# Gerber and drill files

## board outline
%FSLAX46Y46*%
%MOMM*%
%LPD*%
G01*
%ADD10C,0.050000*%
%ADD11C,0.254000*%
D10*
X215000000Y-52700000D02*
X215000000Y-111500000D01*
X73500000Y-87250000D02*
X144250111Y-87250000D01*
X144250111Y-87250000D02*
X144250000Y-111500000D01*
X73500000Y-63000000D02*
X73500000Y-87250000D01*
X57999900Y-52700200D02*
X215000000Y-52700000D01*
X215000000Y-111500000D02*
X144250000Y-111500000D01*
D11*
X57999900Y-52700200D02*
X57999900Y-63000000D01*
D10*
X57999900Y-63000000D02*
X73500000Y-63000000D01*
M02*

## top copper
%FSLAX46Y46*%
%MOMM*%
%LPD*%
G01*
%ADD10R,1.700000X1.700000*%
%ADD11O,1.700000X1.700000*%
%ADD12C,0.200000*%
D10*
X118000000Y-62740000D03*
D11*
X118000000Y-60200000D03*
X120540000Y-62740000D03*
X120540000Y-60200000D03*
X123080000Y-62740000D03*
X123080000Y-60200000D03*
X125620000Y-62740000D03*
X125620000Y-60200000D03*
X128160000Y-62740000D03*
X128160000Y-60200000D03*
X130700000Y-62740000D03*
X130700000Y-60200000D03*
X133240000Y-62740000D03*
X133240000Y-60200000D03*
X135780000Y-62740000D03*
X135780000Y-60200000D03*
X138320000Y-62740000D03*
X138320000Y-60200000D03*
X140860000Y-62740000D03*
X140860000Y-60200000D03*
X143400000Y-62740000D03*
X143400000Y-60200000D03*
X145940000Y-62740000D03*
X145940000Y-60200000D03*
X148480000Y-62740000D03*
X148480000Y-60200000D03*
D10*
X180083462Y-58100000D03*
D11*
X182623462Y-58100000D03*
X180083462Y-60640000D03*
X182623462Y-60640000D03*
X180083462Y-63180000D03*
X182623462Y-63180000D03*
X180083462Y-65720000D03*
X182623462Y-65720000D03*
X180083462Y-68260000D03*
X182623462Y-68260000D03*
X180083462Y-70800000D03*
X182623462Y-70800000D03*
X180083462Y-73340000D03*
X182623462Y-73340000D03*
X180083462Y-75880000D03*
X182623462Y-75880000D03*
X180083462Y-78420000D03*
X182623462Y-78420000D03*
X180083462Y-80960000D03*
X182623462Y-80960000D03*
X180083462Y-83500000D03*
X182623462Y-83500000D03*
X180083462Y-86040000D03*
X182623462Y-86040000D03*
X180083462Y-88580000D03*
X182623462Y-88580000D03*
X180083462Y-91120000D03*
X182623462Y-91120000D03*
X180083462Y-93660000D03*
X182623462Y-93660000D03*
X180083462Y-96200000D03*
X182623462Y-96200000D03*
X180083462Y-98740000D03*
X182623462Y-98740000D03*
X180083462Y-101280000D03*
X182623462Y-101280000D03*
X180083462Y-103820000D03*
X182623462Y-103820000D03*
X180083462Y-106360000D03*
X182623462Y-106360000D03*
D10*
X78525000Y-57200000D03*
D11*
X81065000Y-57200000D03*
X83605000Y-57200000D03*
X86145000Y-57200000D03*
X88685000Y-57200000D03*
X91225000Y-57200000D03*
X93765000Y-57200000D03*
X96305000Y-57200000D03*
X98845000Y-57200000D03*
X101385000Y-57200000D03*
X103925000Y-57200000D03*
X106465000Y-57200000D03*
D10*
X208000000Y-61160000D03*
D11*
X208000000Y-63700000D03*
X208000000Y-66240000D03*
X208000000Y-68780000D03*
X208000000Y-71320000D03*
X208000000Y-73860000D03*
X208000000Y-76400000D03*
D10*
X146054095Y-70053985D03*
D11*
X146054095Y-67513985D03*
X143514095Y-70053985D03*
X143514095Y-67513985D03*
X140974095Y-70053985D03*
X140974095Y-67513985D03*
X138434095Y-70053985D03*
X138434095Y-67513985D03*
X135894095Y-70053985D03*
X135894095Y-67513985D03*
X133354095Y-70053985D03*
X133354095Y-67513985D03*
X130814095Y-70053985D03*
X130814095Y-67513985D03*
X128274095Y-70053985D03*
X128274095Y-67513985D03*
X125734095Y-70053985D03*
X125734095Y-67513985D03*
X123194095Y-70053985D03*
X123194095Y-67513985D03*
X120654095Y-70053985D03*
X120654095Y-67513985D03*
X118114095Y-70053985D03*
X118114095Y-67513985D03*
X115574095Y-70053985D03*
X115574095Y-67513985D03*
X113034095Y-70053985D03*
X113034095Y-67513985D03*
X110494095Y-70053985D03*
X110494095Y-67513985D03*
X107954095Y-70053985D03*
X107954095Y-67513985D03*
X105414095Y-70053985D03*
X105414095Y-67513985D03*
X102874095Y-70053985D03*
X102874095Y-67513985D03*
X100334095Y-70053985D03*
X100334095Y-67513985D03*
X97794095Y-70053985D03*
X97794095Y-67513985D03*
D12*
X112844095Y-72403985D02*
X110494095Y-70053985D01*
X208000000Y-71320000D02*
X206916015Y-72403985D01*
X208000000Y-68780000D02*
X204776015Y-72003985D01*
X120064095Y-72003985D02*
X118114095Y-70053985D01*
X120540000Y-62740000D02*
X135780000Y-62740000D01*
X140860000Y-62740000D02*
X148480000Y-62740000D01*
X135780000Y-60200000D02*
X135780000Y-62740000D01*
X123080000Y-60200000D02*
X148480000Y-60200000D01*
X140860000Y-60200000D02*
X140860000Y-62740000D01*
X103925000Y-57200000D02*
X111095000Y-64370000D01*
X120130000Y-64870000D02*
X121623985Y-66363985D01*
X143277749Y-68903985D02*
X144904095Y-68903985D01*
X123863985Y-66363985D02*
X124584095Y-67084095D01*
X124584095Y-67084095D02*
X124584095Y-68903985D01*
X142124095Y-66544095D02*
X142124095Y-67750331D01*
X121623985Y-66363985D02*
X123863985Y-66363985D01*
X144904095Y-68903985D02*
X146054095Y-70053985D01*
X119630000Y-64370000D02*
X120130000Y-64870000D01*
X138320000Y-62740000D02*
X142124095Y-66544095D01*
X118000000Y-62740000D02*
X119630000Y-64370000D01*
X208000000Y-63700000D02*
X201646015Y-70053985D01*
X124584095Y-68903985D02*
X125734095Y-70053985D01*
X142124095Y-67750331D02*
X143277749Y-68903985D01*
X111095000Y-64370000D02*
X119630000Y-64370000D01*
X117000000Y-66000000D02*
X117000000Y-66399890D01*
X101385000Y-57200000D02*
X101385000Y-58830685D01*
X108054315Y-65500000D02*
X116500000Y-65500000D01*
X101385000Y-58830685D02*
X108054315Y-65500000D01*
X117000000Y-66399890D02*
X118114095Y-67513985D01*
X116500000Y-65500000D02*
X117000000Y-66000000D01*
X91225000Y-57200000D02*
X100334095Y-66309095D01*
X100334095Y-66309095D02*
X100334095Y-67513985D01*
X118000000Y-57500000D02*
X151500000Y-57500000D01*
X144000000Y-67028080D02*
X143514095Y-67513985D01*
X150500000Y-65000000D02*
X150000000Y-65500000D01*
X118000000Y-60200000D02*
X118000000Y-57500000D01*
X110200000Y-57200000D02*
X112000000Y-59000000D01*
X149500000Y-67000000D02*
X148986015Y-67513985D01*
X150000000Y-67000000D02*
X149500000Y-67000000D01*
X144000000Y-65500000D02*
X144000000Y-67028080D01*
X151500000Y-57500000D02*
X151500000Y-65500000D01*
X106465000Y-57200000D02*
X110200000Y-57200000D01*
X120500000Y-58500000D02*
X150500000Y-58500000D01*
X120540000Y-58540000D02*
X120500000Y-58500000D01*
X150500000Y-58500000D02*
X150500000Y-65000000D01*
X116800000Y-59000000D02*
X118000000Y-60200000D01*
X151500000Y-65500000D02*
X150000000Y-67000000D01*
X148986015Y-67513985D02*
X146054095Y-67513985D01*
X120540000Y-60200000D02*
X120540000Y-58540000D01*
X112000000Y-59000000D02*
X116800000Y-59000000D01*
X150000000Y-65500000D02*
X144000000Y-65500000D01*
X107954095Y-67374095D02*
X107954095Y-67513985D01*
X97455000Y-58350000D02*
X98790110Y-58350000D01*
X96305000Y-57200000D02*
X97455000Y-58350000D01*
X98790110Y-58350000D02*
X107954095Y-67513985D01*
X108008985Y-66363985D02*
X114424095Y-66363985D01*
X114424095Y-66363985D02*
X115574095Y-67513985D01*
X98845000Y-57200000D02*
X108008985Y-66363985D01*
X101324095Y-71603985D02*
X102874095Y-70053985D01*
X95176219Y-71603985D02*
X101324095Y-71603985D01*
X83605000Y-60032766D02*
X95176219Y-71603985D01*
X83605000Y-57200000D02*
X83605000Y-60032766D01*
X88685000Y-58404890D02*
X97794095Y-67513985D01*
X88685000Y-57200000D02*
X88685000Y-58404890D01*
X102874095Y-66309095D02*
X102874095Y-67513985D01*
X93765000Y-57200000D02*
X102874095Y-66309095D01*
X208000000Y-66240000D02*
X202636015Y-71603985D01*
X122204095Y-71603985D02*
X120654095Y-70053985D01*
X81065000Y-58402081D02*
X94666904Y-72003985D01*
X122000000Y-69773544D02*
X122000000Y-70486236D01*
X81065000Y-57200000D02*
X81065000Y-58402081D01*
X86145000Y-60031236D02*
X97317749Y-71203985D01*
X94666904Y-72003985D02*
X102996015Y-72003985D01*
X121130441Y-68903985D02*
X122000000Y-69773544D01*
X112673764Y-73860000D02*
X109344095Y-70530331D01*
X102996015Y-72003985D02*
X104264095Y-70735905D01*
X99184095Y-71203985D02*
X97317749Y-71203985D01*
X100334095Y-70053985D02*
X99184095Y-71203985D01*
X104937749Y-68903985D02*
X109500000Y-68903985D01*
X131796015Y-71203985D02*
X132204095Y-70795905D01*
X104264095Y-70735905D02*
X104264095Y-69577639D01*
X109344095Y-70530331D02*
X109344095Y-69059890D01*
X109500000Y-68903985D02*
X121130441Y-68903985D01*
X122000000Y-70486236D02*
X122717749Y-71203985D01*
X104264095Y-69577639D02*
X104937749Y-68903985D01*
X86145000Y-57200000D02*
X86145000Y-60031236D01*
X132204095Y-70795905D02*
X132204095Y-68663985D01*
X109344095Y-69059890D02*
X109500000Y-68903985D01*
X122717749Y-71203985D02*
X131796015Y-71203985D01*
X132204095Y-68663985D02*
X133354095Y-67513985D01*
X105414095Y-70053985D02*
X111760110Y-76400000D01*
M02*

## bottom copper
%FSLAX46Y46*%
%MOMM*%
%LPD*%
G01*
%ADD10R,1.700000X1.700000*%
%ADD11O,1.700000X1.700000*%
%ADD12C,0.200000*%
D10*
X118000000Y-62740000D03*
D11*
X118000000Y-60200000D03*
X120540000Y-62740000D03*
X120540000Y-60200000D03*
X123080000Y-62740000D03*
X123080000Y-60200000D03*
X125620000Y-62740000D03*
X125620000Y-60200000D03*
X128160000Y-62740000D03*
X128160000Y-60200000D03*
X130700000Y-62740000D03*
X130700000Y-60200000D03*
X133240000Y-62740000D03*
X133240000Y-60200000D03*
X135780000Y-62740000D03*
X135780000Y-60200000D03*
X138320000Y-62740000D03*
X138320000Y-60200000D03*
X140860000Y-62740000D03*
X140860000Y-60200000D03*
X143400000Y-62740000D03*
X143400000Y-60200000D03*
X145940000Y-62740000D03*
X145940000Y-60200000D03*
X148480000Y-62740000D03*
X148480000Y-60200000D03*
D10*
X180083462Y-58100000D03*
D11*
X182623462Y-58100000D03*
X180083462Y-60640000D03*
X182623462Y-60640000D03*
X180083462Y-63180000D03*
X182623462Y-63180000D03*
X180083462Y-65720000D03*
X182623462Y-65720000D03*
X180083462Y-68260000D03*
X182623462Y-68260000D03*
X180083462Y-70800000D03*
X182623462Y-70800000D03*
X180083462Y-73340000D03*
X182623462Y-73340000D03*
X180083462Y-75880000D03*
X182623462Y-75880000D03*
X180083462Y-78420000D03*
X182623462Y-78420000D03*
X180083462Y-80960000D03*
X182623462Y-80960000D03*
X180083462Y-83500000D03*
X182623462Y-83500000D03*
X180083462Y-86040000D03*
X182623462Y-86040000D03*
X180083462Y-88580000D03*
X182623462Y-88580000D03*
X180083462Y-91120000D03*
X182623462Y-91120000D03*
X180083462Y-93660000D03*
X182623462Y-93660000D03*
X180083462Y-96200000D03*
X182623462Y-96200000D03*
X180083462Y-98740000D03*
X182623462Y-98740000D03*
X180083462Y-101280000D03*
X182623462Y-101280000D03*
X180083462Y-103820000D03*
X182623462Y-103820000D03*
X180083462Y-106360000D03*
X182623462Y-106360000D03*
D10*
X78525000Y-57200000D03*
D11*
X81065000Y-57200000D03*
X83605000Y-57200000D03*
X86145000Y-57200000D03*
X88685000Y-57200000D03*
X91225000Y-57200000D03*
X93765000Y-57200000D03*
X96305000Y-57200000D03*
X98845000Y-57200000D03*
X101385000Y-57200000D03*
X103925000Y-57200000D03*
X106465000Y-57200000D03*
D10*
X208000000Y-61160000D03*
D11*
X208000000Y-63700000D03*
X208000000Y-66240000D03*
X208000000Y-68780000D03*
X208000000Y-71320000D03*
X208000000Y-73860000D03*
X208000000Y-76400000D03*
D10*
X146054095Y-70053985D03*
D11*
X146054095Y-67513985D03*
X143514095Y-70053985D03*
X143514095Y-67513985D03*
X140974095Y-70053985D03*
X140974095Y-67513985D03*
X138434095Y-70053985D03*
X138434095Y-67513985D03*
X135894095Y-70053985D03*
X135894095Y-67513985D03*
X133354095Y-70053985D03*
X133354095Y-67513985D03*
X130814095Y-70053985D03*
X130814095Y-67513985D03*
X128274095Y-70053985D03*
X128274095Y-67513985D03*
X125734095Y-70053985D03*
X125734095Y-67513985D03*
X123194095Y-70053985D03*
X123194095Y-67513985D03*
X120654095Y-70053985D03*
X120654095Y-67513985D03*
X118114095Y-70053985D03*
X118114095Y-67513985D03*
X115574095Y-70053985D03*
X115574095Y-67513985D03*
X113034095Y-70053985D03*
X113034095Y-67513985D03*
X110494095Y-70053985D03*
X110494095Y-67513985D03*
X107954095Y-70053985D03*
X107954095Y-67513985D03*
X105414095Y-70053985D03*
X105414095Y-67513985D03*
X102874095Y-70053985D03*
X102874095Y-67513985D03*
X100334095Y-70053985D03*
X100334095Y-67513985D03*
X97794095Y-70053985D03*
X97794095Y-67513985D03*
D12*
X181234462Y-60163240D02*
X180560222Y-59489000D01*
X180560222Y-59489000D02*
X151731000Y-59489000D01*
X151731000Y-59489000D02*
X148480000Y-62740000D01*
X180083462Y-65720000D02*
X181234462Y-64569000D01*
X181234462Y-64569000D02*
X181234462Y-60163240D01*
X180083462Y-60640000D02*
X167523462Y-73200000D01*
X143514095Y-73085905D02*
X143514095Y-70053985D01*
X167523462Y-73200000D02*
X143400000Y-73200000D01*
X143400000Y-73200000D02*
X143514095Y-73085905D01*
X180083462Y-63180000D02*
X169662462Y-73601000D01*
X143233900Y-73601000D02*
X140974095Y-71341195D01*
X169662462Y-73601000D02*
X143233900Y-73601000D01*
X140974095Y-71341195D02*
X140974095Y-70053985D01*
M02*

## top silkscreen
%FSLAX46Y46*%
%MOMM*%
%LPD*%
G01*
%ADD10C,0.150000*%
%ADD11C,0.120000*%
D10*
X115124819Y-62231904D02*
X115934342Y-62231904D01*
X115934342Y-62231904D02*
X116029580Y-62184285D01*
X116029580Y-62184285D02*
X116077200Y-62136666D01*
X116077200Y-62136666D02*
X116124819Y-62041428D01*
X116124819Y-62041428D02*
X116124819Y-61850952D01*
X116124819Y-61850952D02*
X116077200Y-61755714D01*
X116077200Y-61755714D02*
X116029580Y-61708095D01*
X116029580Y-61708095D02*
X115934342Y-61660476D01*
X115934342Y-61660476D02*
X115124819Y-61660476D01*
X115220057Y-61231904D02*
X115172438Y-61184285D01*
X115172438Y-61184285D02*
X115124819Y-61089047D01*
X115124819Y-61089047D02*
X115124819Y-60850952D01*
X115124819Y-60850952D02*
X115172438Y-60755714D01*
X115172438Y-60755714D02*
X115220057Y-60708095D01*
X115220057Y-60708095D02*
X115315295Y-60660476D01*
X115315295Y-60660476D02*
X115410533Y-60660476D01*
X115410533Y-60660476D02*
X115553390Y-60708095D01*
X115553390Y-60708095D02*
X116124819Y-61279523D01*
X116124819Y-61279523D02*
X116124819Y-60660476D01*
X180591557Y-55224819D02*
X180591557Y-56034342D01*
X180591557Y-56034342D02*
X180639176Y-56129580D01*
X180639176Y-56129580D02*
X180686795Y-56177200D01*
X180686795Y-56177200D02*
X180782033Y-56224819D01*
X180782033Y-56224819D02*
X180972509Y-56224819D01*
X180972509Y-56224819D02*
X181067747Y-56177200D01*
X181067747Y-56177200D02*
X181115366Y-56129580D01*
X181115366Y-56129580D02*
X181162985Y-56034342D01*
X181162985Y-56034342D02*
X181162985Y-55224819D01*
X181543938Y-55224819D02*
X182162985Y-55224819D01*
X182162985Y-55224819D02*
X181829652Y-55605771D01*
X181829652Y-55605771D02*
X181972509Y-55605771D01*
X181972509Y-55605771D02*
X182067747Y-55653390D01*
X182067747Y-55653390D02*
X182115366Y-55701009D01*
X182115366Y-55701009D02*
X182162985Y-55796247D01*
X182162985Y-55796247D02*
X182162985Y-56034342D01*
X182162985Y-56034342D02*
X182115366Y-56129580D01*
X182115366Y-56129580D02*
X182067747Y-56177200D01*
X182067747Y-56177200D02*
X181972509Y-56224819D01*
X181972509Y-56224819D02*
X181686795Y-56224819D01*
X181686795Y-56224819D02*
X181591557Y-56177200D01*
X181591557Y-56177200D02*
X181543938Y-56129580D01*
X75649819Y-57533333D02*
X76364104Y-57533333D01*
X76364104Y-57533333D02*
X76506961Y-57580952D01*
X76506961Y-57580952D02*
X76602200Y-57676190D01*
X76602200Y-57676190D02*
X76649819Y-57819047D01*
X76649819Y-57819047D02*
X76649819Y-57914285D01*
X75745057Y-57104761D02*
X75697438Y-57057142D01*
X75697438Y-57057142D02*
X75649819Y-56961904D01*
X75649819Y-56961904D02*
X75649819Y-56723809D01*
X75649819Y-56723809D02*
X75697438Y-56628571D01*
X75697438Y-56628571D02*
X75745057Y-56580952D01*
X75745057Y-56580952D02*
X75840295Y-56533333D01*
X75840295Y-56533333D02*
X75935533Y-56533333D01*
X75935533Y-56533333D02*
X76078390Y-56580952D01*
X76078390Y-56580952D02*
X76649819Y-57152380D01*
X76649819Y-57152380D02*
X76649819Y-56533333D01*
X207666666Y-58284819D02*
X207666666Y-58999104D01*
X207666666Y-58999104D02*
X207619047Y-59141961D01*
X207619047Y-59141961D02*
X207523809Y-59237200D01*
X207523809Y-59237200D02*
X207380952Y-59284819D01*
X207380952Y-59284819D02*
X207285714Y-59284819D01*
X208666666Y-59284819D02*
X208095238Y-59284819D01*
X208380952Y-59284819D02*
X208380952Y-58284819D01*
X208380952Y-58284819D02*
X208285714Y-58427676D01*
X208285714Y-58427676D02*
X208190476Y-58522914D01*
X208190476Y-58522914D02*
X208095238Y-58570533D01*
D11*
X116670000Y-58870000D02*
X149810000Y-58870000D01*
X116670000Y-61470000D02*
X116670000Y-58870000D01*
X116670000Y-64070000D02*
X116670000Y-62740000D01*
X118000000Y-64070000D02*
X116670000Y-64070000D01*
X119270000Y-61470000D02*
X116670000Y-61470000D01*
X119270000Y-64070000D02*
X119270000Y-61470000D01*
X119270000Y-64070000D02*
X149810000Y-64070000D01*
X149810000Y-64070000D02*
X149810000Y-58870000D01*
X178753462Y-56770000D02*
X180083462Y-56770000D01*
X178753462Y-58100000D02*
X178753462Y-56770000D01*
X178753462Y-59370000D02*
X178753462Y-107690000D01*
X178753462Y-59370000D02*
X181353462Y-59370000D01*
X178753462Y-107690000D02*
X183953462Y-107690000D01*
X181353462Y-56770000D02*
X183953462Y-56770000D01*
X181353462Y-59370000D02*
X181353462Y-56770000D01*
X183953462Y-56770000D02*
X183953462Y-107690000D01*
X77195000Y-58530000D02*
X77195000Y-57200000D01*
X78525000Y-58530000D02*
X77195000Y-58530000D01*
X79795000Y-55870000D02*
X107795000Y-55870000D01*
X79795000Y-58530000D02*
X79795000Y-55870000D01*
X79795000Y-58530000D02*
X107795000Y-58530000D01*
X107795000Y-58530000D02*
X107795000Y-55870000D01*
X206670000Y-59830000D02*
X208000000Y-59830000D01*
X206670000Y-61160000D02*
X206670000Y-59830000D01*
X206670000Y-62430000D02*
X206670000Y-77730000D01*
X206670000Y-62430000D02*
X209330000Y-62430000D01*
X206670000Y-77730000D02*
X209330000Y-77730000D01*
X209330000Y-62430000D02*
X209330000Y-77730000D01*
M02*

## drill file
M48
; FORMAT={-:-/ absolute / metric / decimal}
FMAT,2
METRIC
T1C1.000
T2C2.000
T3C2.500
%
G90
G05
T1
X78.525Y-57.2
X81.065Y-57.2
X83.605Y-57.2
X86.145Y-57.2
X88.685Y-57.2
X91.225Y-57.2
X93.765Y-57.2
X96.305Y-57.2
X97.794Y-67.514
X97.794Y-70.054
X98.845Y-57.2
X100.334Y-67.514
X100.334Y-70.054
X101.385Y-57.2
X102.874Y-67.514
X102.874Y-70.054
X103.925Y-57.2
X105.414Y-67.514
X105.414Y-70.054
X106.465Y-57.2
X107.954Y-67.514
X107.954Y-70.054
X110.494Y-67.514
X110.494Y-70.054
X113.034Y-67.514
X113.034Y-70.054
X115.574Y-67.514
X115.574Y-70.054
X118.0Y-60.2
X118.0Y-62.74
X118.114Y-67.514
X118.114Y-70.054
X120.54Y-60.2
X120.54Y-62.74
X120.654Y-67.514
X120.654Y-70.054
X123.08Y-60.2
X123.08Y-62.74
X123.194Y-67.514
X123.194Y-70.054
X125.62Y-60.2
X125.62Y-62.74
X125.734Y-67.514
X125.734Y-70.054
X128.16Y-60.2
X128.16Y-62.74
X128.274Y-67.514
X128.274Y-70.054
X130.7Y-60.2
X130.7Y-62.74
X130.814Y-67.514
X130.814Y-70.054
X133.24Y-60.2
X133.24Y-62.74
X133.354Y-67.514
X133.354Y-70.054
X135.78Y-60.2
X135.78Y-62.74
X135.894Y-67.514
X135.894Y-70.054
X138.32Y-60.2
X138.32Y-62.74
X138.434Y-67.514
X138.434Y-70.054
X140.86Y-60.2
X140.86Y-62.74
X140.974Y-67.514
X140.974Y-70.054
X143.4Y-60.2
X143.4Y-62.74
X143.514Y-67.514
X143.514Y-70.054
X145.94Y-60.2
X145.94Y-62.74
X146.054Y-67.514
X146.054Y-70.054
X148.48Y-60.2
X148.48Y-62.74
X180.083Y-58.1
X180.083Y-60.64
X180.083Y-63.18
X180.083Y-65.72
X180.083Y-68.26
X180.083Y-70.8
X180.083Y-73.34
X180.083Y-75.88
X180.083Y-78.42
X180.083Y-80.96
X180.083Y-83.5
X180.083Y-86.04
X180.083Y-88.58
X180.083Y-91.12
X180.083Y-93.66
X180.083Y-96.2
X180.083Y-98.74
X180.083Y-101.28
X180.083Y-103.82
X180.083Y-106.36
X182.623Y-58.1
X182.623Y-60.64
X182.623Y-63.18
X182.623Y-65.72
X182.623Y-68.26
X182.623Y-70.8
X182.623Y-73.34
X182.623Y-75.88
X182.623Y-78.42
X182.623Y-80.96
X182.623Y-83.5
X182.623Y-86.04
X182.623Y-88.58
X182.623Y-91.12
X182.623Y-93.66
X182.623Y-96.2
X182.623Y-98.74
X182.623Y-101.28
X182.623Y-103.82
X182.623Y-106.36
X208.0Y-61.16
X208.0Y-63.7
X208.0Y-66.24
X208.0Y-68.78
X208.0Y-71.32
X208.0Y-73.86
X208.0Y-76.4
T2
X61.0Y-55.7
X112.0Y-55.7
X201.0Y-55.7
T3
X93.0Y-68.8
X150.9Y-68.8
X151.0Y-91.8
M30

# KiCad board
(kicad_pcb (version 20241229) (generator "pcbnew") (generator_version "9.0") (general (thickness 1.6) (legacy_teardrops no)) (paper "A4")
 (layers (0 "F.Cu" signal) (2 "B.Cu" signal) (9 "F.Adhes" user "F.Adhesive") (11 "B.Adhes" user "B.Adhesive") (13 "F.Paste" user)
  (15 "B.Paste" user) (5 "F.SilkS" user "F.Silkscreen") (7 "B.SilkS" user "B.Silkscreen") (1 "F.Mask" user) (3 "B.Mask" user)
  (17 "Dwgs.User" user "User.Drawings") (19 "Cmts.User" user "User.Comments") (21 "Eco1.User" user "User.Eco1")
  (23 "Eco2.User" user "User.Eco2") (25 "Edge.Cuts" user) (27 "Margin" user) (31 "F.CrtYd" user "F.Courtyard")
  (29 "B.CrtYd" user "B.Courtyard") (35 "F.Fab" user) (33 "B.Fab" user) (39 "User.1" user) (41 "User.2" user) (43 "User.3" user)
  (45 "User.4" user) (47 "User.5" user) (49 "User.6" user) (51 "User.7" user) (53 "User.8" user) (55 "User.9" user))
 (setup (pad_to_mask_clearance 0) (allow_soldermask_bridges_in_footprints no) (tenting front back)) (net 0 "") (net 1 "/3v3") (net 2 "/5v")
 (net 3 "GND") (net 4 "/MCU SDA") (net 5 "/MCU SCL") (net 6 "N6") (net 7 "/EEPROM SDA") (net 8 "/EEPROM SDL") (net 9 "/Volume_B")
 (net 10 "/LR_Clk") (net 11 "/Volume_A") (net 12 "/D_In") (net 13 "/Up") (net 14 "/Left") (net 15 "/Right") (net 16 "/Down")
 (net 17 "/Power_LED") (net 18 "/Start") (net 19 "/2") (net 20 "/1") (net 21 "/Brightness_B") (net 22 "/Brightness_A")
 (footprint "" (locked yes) (layer "F.Cu") (at 151 91.8)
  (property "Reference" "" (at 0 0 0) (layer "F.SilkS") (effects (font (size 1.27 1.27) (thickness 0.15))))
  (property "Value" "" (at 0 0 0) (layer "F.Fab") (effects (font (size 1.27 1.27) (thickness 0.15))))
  (pad "" np_thru_hole circle (at 0 0 180) (size 2.5 2.5) (drill 2.5) (layers "*.Cu" "*.Mask")))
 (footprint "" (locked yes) (layer "F.Cu") (at 112 55.7)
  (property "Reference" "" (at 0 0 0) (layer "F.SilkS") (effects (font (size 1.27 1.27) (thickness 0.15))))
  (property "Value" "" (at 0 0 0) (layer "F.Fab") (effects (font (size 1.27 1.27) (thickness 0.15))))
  (pad "" np_thru_hole circle (at 0 0 180) (size 2 2) (drill 2) (layers "*.Cu" "*.Mask")))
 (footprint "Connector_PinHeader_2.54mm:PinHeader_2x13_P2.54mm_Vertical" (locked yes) (layer "F.Cu") (at 118 62.74 90)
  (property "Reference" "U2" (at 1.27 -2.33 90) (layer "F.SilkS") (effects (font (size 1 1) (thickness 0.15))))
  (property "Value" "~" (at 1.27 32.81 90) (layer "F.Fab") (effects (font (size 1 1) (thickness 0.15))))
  (fp_line (start 3.87 -1.33) (end 3.87 31.81) (stroke (width 0.12) (type solid)) (layer "F.SilkS"))
  (fp_line (start 1.27 -1.33) (end 3.87 -1.33) (stroke (width 0.12) (type solid)) (layer "F.SilkS"))
  (fp_line (start -1.33 -1.33) (end 0 -1.33) (stroke (width 0.12) (type solid)) (layer "F.SilkS"))
  (fp_line (start -1.33 0) (end -1.33 -1.33) (stroke (width 0.12) (type solid)) (layer "F.SilkS"))
  (fp_line (start 1.27 1.27) (end 1.27 -1.33) (stroke (width 0.12) (type solid)) (layer "F.SilkS"))
  (fp_line (start -1.33 1.27) (end 1.27 1.27) (stroke (width 0.12) (type solid)) (layer "F.SilkS"))
  (fp_line (start -1.33 1.27) (end -1.33 31.81) (stroke (width 0.12) (type solid)) (layer "F.SilkS"))
  (fp_line (start -1.33 31.81) (end 3.87 31.81) (stroke (width 0.12) (type solid)) (layer "F.SilkS"))
  (pad "1" thru_hole rect (at 0 0 90) (size 1.7 1.7) (drill 1) (layers "*.Cu" "*.Mask") (remove_unused_layers no) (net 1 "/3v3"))
  (pad "2" thru_hole oval (at 2.54 0 90) (size 1.7 1.7) (drill 1) (layers "*.Cu" "*.Mask") (remove_unused_layers no) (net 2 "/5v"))
  (pad "3" thru_hole oval (at 0 2.54 90) (size 1.7 1.7) (drill 1) (layers "*.Cu" "*.Mask") (remove_unused_layers no) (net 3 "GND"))
  (pad "4" thru_hole oval (at 2.54 2.54 90) (size 1.7 1.7) (drill 1) (layers "*.Cu" "*.Mask") (remove_unused_layers no) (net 2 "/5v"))
  (pad "5" thru_hole oval (at 0 5.08 90) (size 1.7 1.7) (drill 1) (layers "*.Cu" "*.Mask") (remove_unused_layers no) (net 3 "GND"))
  (pad "6" thru_hole oval (at 2.54 5.08 90) (size 1.7 1.7) (drill 1) (layers "*.Cu" "*.Mask") (remove_unused_layers no) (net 3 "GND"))
  (pad "7" thru_hole oval (at 0 7.62 90) (size 1.7 1.7) (drill 1) (layers "*.Cu" "*.Mask") (remove_unused_layers no) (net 3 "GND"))
  (pad "8" thru_hole oval (at 2.54 7.62 90) (size 1.7 1.7) (drill 1) (layers "*.Cu" "*.Mask") (remove_unused_layers no) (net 3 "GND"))
  (pad "9" thru_hole oval (at 0 10.16 90) (size 1.7 1.7) (drill 1) (layers "*.Cu" "*.Mask") (remove_unused_layers no) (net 3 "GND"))
  (pad "10" thru_hole oval (at 2.54 10.16 90) (size 1.7 1.7) (drill 1) (layers "*.Cu" "*.Mask") (remove_unused_layers no) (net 3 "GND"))
  (pad "11" thru_hole oval (at 0 12.7 90) (size 1.7 1.7) (drill 1) (layers "*.Cu" "*.Mask") (remove_unused_layers no) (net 3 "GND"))
  (pad "12" thru_hole oval (at 2.54 12.7 90) (size 1.7 1.7) (drill 1) (layers "*.Cu" "*.Mask") (remove_unused_layers no) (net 3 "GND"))
  (pad "13" thru_hole oval (at 0 15.24 90) (size 1.7 1.7) (drill 1) (layers "*.Cu" "*.Mask") (remove_unused_layers no) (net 3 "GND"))
  (pad "14" thru_hole oval (at 2.54 15.24 90) (size 1.7 1.7) (drill 1) (layers "*.Cu" "*.Mask") (remove_unused_layers no) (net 3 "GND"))
  (pad "15" thru_hole oval (at 0 17.78 90) (size 1.7 1.7) (drill 1) (layers "*.Cu" "*.Mask") (remove_unused_layers no) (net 3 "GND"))
  (pad "16" thru_hole oval (at 2.54 17.78 90) (size 1.7 1.7) (drill 1) (layers "*.Cu" "*.Mask") (remove_unused_layers no) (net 3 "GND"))
  (pad "17" thru_hole oval (at 0 20.32 90) (size 1.7 1.7) (drill 1) (layers "*.Cu" "*.Mask") (remove_unused_layers no) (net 1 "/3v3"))
  (pad "18" thru_hole oval (at 2.54 20.32 90) (size 1.7 1.7) (drill 1) (layers "*.Cu" "*.Mask") (remove_unused_layers no) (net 3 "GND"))
  (pad "19" thru_hole oval (at 0 22.86 90) (size 1.7 1.7) (drill 1) (layers "*.Cu" "*.Mask") (remove_unused_layers no) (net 3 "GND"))
  (pad "20" thru_hole oval (at 2.54 22.86 90) (size 1.7 1.7) (drill 1) (layers "*.Cu" "*.Mask") (remove_unused_layers no) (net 3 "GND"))
  (pad "21" thru_hole oval (at 0 25.4 90) (size 1.7 1.7) (drill 1) (layers "*.Cu" "*.Mask") (remove_unused_layers no) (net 3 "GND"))
  (pad "22" thru_hole oval (at 2.54 25.4 90) (size 1.7 1.7) (drill 1) (layers "*.Cu" "*.Mask") (remove_unused_layers no) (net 3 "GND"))
  (pad "23" thru_hole oval (at 0 27.94 90) (size 1.7 1.7) (drill 1) (layers "*.Cu" "*.Mask") (remove_unused_layers no) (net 3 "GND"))
  (pad "24" thru_hole oval (at 2.54 27.94 90) (size 1.7 1.7) (drill 1) (layers "*.Cu" "*.Mask") (remove_unused_layers no) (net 3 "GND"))
  (pad "25" thru_hole oval (at 0 30.48 90) (size 1.7 1.7) (drill 1) (layers "*.Cu" "*.Mask") (remove_unused_layers no) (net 3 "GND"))
  (pad "26" thru_hole oval (at 2.54 30.48 90) (size 1.7 1.7) (drill 1) (layers "*.Cu" "*.Mask") (remove_unused_layers no) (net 3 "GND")))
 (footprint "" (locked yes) (layer "F.Cu") (at 93 68.8)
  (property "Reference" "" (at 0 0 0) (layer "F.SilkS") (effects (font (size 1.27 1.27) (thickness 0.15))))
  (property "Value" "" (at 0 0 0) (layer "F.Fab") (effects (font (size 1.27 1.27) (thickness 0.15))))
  (pad "" np_thru_hole circle (at 0 0 180) (size 2.5 2.5) (drill 2.5) (layers "*.Cu" "*.Mask")))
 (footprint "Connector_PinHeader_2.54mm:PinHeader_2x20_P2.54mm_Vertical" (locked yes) (layer "F.Cu") (at 180.083462 58.1)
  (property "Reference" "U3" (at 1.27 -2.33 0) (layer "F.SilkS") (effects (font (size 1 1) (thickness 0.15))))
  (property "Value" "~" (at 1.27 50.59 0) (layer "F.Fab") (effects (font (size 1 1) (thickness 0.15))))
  (fp_line (start -1.33 -1.33) (end 0 -1.33) (stroke (width 0.12) (type solid)) (layer "F.SilkS"))
  (fp_line (start -1.33 0) (end -1.33 -1.33) (stroke (width 0.12) (type solid)) (layer "F.SilkS"))
  (fp_line (start -1.33 1.27) (end -1.33 49.59) (stroke (width 0.12) (type solid)) (layer "F.SilkS"))
  (fp_line (start -1.33 1.27) (end 1.27 1.27) (stroke (width 0.12) (type solid)) (layer "F.SilkS"))
  (fp_line (start -1.33 49.59) (end 3.87 49.59) (stroke (width 0.12) (type solid)) (layer "F.SilkS"))
  (fp_line (start 1.27 -1.33) (end 3.87 -1.33) (stroke (width 0.12) (type solid)) (layer "F.SilkS"))
  (fp_line (start 1.27 1.27) (end 1.27 -1.33) (stroke (width 0.12) (type solid)) (layer "F.SilkS"))
  (fp_line (start 3.87 -1.33) (end 3.87 49.59) (stroke (width 0.12) (type solid)) (layer "F.SilkS"))
  (pad "1" thru_hole rect (at 0 0) (size 1.7 1.7) (drill 1) (layers "*.Cu" "*.Mask") (remove_unused_layers no) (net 1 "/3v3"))
  (pad "2" thru_hole oval (at 2.54 0) (size 1.7 1.7) (drill 1) (layers "*.Cu" "*.Mask") (remove_unused_layers no) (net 2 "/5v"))
  (pad "3" thru_hole oval (at 0 2.54) (size 1.7 1.7) (drill 1) (layers "*.Cu" "*.Mask") (remove_unused_layers no) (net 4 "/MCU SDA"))
  (pad "4" thru_hole oval (at 2.54 2.54) (size 1.7 1.7) (drill 1) (layers "*.Cu" "*.Mask") (remove_unused_layers no) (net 2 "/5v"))
  (pad "5" thru_hole oval (at 0 5.08) (size 1.7 1.7) (drill 1) (layers "*.Cu" "*.Mask") (remove_unused_layers no) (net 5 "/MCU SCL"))
  (pad "6" thru_hole oval (at 2.54 5.08) (size 1.7 1.7) (drill 1) (layers "*.Cu" "*.Mask") (remove_unused_layers no) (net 3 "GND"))
  (pad "7" thru_hole oval (at 0 7.62) (size 1.7 1.7) (drill 1) (layers "*.Cu" "*.Mask") (remove_unused_layers no) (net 3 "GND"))
  (pad "8" thru_hole oval (at 2.54 7.62) (size 1.7 1.7) (drill 1) (layers "*.Cu" "*.Mask") (remove_unused_layers no) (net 3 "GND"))
  (pad "9" thru_hole oval (at 0 10.16) (size 1.7 1.7) (drill 1) (layers "*.Cu" "*.Mask") (remove_unused_layers no) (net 3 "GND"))
  (pad "10" thru_hole oval (at 2.54 10.16) (size 1.7 1.7) (drill 1) (layers "*.Cu" "*.Mask") (remove_unused_layers no) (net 3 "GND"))
  (pad "11" thru_hole oval (at 0 12.7) (size 1.7 1.7) (drill 1) (layers "*.Cu" "*.Mask") (remove_unused_layers no) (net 3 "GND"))
  (pad "12" thru_hole oval (at 2.54 12.7) (size 1.7 1.7) (drill 1) (layers "*.Cu" "*.Mask") (remove_unused_layers no) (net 3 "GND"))
  (pad "13" thru_hole oval (at 0 15.24) (size 1.7 1.7) (drill 1) (layers "*.Cu" "*.Mask") (remove_unused_layers no) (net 3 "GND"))
  (pad "14" thru_hole oval (at 2.54 15.24) (size 1.7 1.7) (drill 1) (layers "*.Cu" "*.Mask") (remove_unused_layers no) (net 3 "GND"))
  (pad "15" thru_hole oval (at 0 17.78) (size 1.7 1.7) (drill 1) (layers "*.Cu" "*.Mask") (remove_unused_layers no) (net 3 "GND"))
  (pad "16" thru_hole oval (at 2.54 17.78) (size 1.7 1.7) (drill 1) (layers "*.Cu" "*.Mask") (remove_unused_layers no) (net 3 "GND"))
  (pad "17" thru_hole oval (at 0 20.32) (size 1.7 1.7) (drill 1) (layers "*.Cu" "*.Mask") (remove_unused_layers no) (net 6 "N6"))
  (pad "18" thru_hole oval (at 2.54 20.32) (size 1.7 1.7) (drill 1) (layers "*.Cu" "*.Mask") (remove_unused_layers no) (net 3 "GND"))
  (pad "19" thru_hole oval (at 0 22.86) (size 1.7 1.7) (drill 1) (layers "*.Cu" "*.Mask") (remove_unused_layers no) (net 3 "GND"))
  (pad "20" thru_hole oval (at 2.54 22.86) (size 1.7 1.7) (drill 1) (layers "*.Cu" "*.Mask") (remove_unused_layers no) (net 3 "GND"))
  (pad "21" thru_hole oval (at 0 25.4) (size 1.7 1.7) (drill 1) (layers "*.Cu" "*.Mask") (remove_unused_layers no) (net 3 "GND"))
  (pad "22" thru_hole oval (at 2.54 25.4) (size 1.7 1.7) (drill 1) (layers "*.Cu" "*.Mask") (remove_unused_layers no) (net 3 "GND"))
  (pad "23" thru_hole oval (at 0 27.94) (size 1.7 1.7) (drill 1) (layers "*.Cu" "*.Mask") (remove_unused_layers no) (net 3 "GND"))
  (pad "24" thru_hole oval (at 2.54 27.94) (size 1.7 1.7) (drill 1) (layers "*.Cu" "*.Mask") (remove_unused_layers no) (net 3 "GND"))
  (pad "25" thru_hole oval (at 0 30.48) (size 1.7 1.7) (drill 1) (layers "*.Cu" "*.Mask") (remove_unused_layers no) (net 3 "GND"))
  (pad "26" thru_hole oval (at 2.54 30.48) (size 1.7 1.7) (drill 1) (layers "*.Cu" "*.Mask") (remove_unused_layers no) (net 3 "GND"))
  (pad "27" thru_hole oval (at 0 33.02) (size 1.7 1.7) (drill 1) (layers "*.Cu" "*.Mask") (remove_unused_layers no) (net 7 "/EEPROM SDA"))
  (pad "28" thru_hole oval (at 2.54 33.02) (size 1.7 1.7) (drill 1) (layers "*.Cu" "*.Mask") (remove_unused_layers no) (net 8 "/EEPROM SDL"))
  (pad "29" thru_hole oval (at 0 35.56) (size 1.7 1.7) (drill 1) (layers "*.Cu" "*.Mask") (remove_unused_layers no) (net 3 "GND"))
  (pad "30" thru_hole oval (at 2.54 35.56) (size 1.7 1.7) (drill 1) (layers "*.Cu" "*.Mask") (remove_unused_layers no) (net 3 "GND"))
  (pad "31" thru_hole oval (at 0 38.1) (size 1.7 1.7) (drill 1) (layers "*.Cu" "*.Mask") (remove_unused_layers no) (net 3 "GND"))
  (pad "32" thru_hole oval (at 2.54 38.1) (size 1.7 1.7) (drill 1) (layers "*.Cu" "*.Mask") (remove_unused_layers no) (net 3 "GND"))
  (pad "33" thru_hole oval (at 0 40.64) (size 1.7 1.7) (drill 1) (layers "*.Cu" "*.Mask") (remove_unused_layers no) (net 3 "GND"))
  (pad "34" thru_hole oval (at 2.54 40.64) (size 1.7 1.7) (drill 1) (layers "*.Cu" "*.Mask") (remove_unused_layers no) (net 3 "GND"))
  (pad "35" thru_hole oval (at 0 43.18) (size 1.7 1.7) (drill 1) (layers "*.Cu" "*.Mask") (remove_unused_layers no) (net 3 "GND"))
  (pad "36" thru_hole oval (at 2.54 43.18) (size 1.7 1.7) (drill 1) (layers "*.Cu" "*.Mask") (remove_unused_layers no) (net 3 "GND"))
  (pad "37" thru_hole oval (at 0 45.72) (size 1.7 1.7) (drill 1) (layers "*.Cu" "*.Mask") (remove_unused_layers no) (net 3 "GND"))
  (pad "38" thru_hole oval (at 2.54 45.72) (size 1.7 1.7) (drill 1) (layers "*.Cu" "*.Mask") (remove_unused_layers no) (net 3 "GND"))
  (pad "39" thru_hole oval (at 0 48.26) (size 1.7 1.7) (drill 1) (layers "*.Cu" "*.Mask") (remove_unused_layers no) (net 3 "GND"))
  (pad "40" thru_hole oval (at 2.54 48.26) (size 1.7 1.7) (drill 1) (layers "*.Cu" "*.Mask") (remove_unused_layers no) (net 3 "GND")))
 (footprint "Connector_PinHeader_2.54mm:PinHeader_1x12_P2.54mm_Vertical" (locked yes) (layer "F.Cu") (at 78.525 57.2 90)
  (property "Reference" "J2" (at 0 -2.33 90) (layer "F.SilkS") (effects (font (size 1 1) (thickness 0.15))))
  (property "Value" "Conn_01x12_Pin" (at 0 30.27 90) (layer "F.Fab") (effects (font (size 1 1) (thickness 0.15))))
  (fp_line (start -1.33 -1.33) (end 0 -1.33) (stroke (width 0.12) (type solid)) (layer "F.SilkS"))
  (fp_line (start -1.33 0) (end -1.33 -1.33) (stroke (width 0.12) (type solid)) (layer "F.SilkS"))
  (fp_line (start 1.33 1.27) (end 1.33 29.27) (stroke (width 0.12) (type solid)) (layer "F.SilkS"))
  (fp_line (start -1.33 1.27) (end 1.33 1.27) (stroke (width 0.12) (type solid)) (layer "F.SilkS"))
  (fp_line (start -1.33 1.27) (end -1.33 29.27) (stroke (width 0.12) (type solid)) (layer "F.SilkS"))
  (fp_line (start -1.33 29.27) (end 1.33 29.27) (stroke (width 0.12) (type solid)) (layer "F.SilkS"))
  (pad "1" thru_hole rect (at 0 0 90) (size 1.7 1.7) (drill 1) (layers "*.Cu" "*.Mask") (remove_unused_layers no) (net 3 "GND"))
  (pad "2" thru_hole oval (at 0 2.54 90) (size 1.7 1.7) (drill 1) (layers "*.Cu" "*.Mask") (remove_unused_layers no) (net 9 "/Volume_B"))
  (pad "3" thru_hole oval (at 0 5.08 90) (size 1.7 1.7) (drill 1) (layers "*.Cu" "*.Mask") (remove_unused_layers no) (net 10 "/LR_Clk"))
  (pad "4" thru_hole oval (at 0 7.62 90) (size 1.7 1.7) (drill 1) (layers "*.Cu" "*.Mask") (remove_unused_layers no) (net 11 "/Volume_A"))
  (pad "5" thru_hole oval (at 0 10.16 90) (size 1.7 1.7) (drill 1) (layers "*.Cu" "*.Mask") (remove_unused_layers no) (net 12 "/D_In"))
  (pad "6" thru_hole oval (at 0 12.7 90) (size 1.7 1.7) (drill 1) (layers "*.Cu" "*.Mask") (remove_unused_layers no) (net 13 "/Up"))
  (pad "7" thru_hole oval (at 0 15.24 90) (size 1.7 1.7) (drill 1) (layers "*.Cu" "*.Mask") (remove_unused_layers no) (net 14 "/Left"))
  (pad "8" thru_hole oval (at 0 17.78 90) (size 1.7 1.7) (drill 1) (layers "*.Cu" "*.Mask") (remove_unused_layers no) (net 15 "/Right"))
  (pad "9" thru_hole oval (at 0 20.32 90) (size 1.7 1.7) (drill 1) (layers "*.Cu" "*.Mask") (remove_unused_layers no) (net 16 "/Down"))
  (pad "10" thru_hole oval (at 0 22.86 90) (size 1.7 1.7) (drill 1) (layers "*.Cu" "*.Mask") (remove_unused_layers no) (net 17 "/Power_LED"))
  (pad "11" thru_hole oval (at 0 25.4 90) (size 1.7 1.7) (drill 1) (layers "*.Cu" "*.Mask") (remove_unused_layers no) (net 1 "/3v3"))
  (pad "12" thru_hole oval (at 0 27.94 90) (size 1.7 1.7) (drill 1) (layers "*.Cu" "*.Mask") (remove_unused_layers no) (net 2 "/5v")))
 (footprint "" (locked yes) (layer "F.Cu") (at 150.9 68.8)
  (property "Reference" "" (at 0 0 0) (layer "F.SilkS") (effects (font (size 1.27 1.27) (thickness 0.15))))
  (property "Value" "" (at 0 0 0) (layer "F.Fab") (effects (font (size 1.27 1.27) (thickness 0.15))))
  (pad "" np_thru_hole circle (at 0 0 180) (size 2.5 2.5) (drill 2.5) (layers "*.Cu" "*.Mask")))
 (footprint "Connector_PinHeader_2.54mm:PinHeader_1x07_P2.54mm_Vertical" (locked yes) (layer "F.Cu") (at 208 61.16)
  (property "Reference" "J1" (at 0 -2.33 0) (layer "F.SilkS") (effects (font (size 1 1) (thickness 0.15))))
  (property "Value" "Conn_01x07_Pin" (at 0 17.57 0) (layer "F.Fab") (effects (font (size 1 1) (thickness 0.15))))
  (fp_line (start -1.33 -1.33) (end 0 -1.33) (stroke (width 0.12) (type solid)) (layer "F.SilkS"))
  (fp_line (start -1.33 0) (end -1.33 -1.33) (stroke (width 0.12) (type solid)) (layer "F.SilkS"))
  (fp_line (start -1.33 1.27) (end -1.33 16.57) (stroke (width 0.12) (type solid)) (layer "F.SilkS"))
  (fp_line (start -1.33 1.27) (end 1.33 1.27) (stroke (width 0.12) (type solid)) (layer "F.SilkS"))
  (fp_line (start -1.33 16.57) (end 1.33 16.57) (stroke (width 0.12) (type solid)) (layer "F.SilkS"))
  (fp_line (start 1.33 1.27) (end 1.33 16.57) (stroke (width 0.12) (type solid)) (layer "F.SilkS"))
  (pad "1" thru_hole rect (at 0 0) (size 1.7 1.7) (drill 1) (layers "*.Cu" "*.Mask") (remove_unused_layers no) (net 3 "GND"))
  (pad "2" thru_hole oval (at 0 2.54) (size 1.7 1.7) (drill 1) (layers "*.Cu" "*.Mask") (remove_unused_layers no) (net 1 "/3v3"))
  (pad "3" thru_hole oval (at 0 5.08) (size 1.7 1.7) (drill 1) (layers "*.Cu" "*.Mask") (remove_unused_layers no) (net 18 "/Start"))
  (pad "4" thru_hole oval (at 0 7.62) (size 1.7 1.7) (drill 1) (layers "*.Cu" "*.Mask") (remove_unused_layers no) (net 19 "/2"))
  (pad "5" thru_hole oval (at 0 10.16) (size 1.7 1.7) (drill 1) (layers "*.Cu" "*.Mask") (remove_unused_layers no) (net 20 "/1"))
  (pad "6" thru_hole oval (at 0 12.7) (size 1.7 1.7) (drill 1) (layers "*.Cu" "*.Mask") (remove_unused_layers no) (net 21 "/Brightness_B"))
  (pad "7" thru_hole oval (at 0 15.24) (size 1.7 1.7) (drill 1) (layers "*.Cu" "*.Mask") (remove_unused_layers no) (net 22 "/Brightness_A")))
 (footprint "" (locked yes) (layer "F.Cu") (at 60.9999 55.6999)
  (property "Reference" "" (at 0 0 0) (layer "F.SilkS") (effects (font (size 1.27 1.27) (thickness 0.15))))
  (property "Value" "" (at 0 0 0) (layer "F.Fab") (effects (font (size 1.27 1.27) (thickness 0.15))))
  (pad "" np_thru_hole circle (at 0 0) (size 2 2) (drill 2) (layers "*.Cu" "*.Mask")))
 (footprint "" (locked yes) (layer "F.Cu") (at 201 55.7)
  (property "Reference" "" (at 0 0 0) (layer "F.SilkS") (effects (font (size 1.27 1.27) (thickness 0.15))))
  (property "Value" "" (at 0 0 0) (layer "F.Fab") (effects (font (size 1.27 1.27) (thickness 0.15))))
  (pad "" np_thru_hole circle (at 0 0 180) (size 2 2) (drill 2) (layers "*.Cu" "*.Mask")))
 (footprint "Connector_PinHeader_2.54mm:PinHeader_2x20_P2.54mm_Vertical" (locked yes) (layer "B.Cu") (at 146.054095 70.053985 90)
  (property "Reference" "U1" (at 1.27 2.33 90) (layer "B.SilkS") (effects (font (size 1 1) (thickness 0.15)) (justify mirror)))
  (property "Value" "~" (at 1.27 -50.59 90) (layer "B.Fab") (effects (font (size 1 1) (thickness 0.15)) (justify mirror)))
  (pad "1" thru_hole rect (at 0 0 90) (size 1.7 1.7) (drill 1) (layers "*.Cu" "*.Mask") (remove_unused_layers no) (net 1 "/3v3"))
  (pad "2" thru_hole oval (at 2.54 0 90) (size 1.7 1.7) (drill 1) (layers "*.Cu" "*.Mask") (remove_unused_layers no) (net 2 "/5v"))
  (pad "3" thru_hole oval (at 0 -2.54 90) (size 1.7 1.7) (drill 1) (layers "*.Cu" "*.Mask") (remove_unused_layers no) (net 4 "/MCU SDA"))
  (pad "4" thru_hole oval (at 2.54 -2.54 90) (size 1.7 1.7) (drill 1) (layers "*.Cu" "*.Mask") (remove_unused_layers no) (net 2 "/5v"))
  (pad "5" thru_hole oval (at 0 -5.08 90) (size 1.7 1.7) (drill 1) (layers "*.Cu" "*.Mask") (remove_unused_layers no) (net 5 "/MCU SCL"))
  (pad "6" thru_hole oval (at 2.54 -5.08 90) (size 1.7 1.7) (drill 1) (layers "*.Cu" "*.Mask") (remove_unused_layers no) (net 3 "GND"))
  (pad "7" thru_hole oval (at 0 -7.62 90) (size 1.7 1.7) (drill 1) (layers "*.Cu" "*.Mask") (remove_unused_layers no) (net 3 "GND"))
  (pad "8" thru_hole oval (at 2.54 -7.62 90) (size 1.7 1.7) (drill 1) (layers "*.Cu" "*.Mask") (remove_unused_layers no) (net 3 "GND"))
  (pad "9" thru_hole oval (at 0 -10.16 90) (size 1.7 1.7) (drill 1) (layers "*.Cu" "*.Mask") (remove_unused_layers no) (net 3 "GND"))
  (pad "10" thru_hole oval (at 2.54 -10.16 90) (size 1.7 1.7) (drill 1) (layers "*.Cu" "*.Mask") (remove_unused_layers no) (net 3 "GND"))
  (pad "11" thru_hole oval (at 0 -12.7 90) (size 1.7 1.7) (drill 1) (layers "*.Cu" "*.Mask") (remove_unused_layers no) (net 3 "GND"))
  (pad "12" thru_hole oval (at 2.54 -12.7 90) (size 1.7 1.7) (drill 1) (layers "*.Cu" "*.Mask") (remove_unused_layers no)
   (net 9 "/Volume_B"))
  (pad "13" thru_hole oval (at 0 -15.24 90) (size 1.7 1.7) (drill 1) (layers "*.Cu" "*.Mask") (remove_unused_layers no) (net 3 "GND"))
  (pad "14" thru_hole oval (at 2.54 -15.24 90) (size 1.7 1.7) (drill 1) (layers "*.Cu" "*.Mask") (remove_unused_layers no) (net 3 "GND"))
  (pad "15" thru_hole oval (at 0 -17.78 90) (size 1.7 1.7) (drill 1) (layers "*.Cu" "*.Mask") (remove_unused_layers no) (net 3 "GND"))
  (pad "16" thru_hole oval (at 2.54 -17.78 90) (size 1.7 1.7) (drill 1) (layers "*.Cu" "*.Mask") (remove_unused_layers no) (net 3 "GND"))
  (pad "17" thru_hole oval (at 0 -20.32 90) (size 1.7 1.7) (drill 1) (layers "*.Cu" "*.Mask") (remove_unused_layers no) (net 1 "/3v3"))
  (pad "18" thru_hole oval (at 2.54 -20.32 90) (size 1.7 1.7) (drill 1) (layers "*.Cu" "*.Mask") (remove_unused_layers no) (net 3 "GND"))
  (pad "19" thru_hole oval (at 0 -22.86 90) (size 1.7 1.7) (drill 1) (layers "*.Cu" "*.Mask") (remove_unused_layers no) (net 3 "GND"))
  (pad "20" thru_hole oval (at 2.54 -22.86 90) (size 1.7 1.7) (drill 1) (layers "*.Cu" "*.Mask") (remove_unused_layers no) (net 3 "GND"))
  (pad "21" thru_hole oval (at 0 -25.4 90) (size 1.7 1.7) (drill 1) (layers "*.Cu" "*.Mask") (remove_unused_layers no) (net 18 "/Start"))
  (pad "22" thru_hole oval (at 2.54 -25.4 90) (size 1.7 1.7) (drill 1) (layers "*.Cu" "*.Mask") (remove_unused_layers no) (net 3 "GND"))
  (pad "23" thru_hole oval (at 0 -27.94 90) (size 1.7 1.7) (drill 1) (layers "*.Cu" "*.Mask") (remove_unused_layers no) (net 19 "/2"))
  (pad "24" thru_hole oval (at 2.54 -27.94 90) (size 1.7 1.7) (drill 1) (layers "*.Cu" "*.Mask") (remove_unused_layers no)
   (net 17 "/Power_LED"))
  (pad "25" thru_hole oval (at 0 -30.48 90) (size 1.7 1.7) (drill 1) (layers "*.Cu" "*.Mask") (remove_unused_layers no) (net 3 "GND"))
  (pad "26" thru_hole oval (at 2.54 -30.48 90) (size 1.7 1.7) (drill 1) (layers "*.Cu" "*.Mask") (remove_unused_layers no) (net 16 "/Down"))
  (pad "27" thru_hole oval (at 0 -33.02 90) (size 1.7 1.7) (drill 1) (layers "*.Cu" "*.Mask") (remove_unused_layers no)
   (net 7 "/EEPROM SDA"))
  (pad "28" thru_hole oval (at 2.54 -33.02 90) (size 1.7 1.7) (drill 1) (layers "*.Cu" "*.Mask") (remove_unused_layers no)
   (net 8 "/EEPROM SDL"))
  (pad "29" thru_hole oval (at 0 -35.56 90) (size 1.7 1.7) (drill 1) (layers "*.Cu" "*.Mask") (remove_unused_layers no) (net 20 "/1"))
  (pad "30" thru_hole oval (at 2.54 -35.56 90) (size 1.7 1.7) (drill 1) (layers "*.Cu" "*.Mask") (remove_unused_layers no) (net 3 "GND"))
  (pad "31" thru_hole oval (at 0 -38.1 90) (size 1.7 1.7) (drill 1) (layers "*.Cu" "*.Mask") (remove_unused_layers no) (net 3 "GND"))
  (pad "32" thru_hole oval (at 2.54 -38.1 90) (size 1.7 1.7) (drill 1) (layers "*.Cu" "*.Mask") (remove_unused_layers no) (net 15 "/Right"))
  (pad "33" thru_hole oval (at 0 -40.64 90) (size 1.7 1.7) (drill 1) (layers "*.Cu" "*.Mask") (remove_unused_layers no)
   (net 22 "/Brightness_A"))
  (pad "34" thru_hole oval (at 2.54 -40.64 90) (size 1.7 1.7) (drill 1) (layers "*.Cu" "*.Mask") (remove_unused_layers no) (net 3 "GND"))
  (pad "35" thru_hole oval (at 0 -43.18 90) (size 1.7 1.7) (drill 1) (layers "*.Cu" "*.Mask") (remove_unused_layers no) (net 10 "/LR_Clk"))
  (pad "36" thru_hole oval (at 2.54 -43.18 90) (size 1.7 1.7) (drill 1) (layers "*.Cu" "*.Mask") (remove_unused_layers no) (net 14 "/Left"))
  (pad "37" thru_hole oval (at 0 -45.72 90) (size 1.7 1.7) (drill 1) (layers "*.Cu" "*.Mask") (remove_unused_layers no) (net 9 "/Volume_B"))
  (pad "38" thru_hole oval (at 2.54 -45.72 90) (size 1.7 1.7) (drill 1) (layers "*.Cu" "*.Mask") (remove_unused_layers no) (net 13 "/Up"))
  (pad "39" thru_hole oval (at 0 -48.26 90) (size 1.7 1.7) (drill 1) (layers "*.Cu" "*.Mask") (remove_unused_layers no) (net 3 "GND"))
  (pad "40" thru_hole oval (at 2.54 -48.26 90) (size 1.7 1.7) (drill 1) (layers "*.Cu" "*.Mask") (remove_unused_layers no) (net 12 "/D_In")))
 (gr_line (start 215 52.7) (end 215 111.5) (stroke (width 0.05) (type default)) (layer "Edge.Cuts"))
 (gr_line (start 73.5 87.25) (end 144.250111 87.25) (stroke (width 0.05) (type default)) (layer "Edge.Cuts"))
 (gr_line (start 144.250111 87.25) (end 144.25 111.5) (stroke (width 0.05) (type default)) (layer "Edge.Cuts"))
 (gr_line (start 73.5 63) (end 73.5 87.25) (stroke (width 0.05) (type default)) (layer "Edge.Cuts"))
 (gr_line (start 57.9999 52.7002) (end 215 52.7) (stroke (width 0.05) (type default)) (layer "Edge.Cuts"))
 (gr_line (start 215 111.5) (end 144.25 111.5) (stroke (width 0.05) (type default)) (layer "Edge.Cuts"))
 (gr_line (start 57.9999 52.7002) (end 57.9999 63) (stroke (width 0.254) (type default)) (layer "Edge.Cuts"))
 (gr_line (start 57.9999 63) (end 73.5 63) (stroke (width 0.05) (type default)) (layer "Edge.Cuts"))
 (segment (start 112.844095 72.403985) (end 110.494095 70.053985) (width 0.2) (layer "F.Cu") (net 20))
 (segment (start 208 71.32) (end 206.916015 72.403985) (width 0.2) (layer "F.Cu") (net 20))
 (segment (start 208 68.78) (end 204.776015 72.003985) (width 0.2) (layer "F.Cu") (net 19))
 (segment (start 120.064095 72.003985) (end 118.114095 70.053985) (width 0.2) (layer "F.Cu") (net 19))
 (segment (start 120.54 62.74) (end 135.78 62.74) (width 0.2) (layer "F.Cu") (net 3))
 (segment (start 140.86 62.74) (end 148.48 62.74) (width 0.2) (layer "F.Cu") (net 3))
 (segment (start 135.78 60.2) (end 135.78 62.74) (width 0.2) (layer "F.Cu") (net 3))
 (segment (start 123.08 60.2) (end 148.48 60.2) (width 0.2) (layer "F.Cu") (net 3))
 (segment (start 140.86 60.2) (end 140.86 62.74) (width 0.2) (layer "F.Cu") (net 3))
 (segment (start 181.234462 60.16324) (end 180.560222 59.489) (width 0.2) (layer "B.Cu") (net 3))
 (segment (start 180.560222 59.489) (end 151.731 59.489) (width 0.2) (layer "B.Cu") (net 3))
 (segment (start 151.731 59.489) (end 148.48 62.74) (width 0.2) (layer "B.Cu") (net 3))
 (segment (start 180.083462 65.72) (end 181.234462 64.569) (width 0.2) (layer "B.Cu") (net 3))
 (segment (start 181.234462 64.569) (end 181.234462 60.16324) (width 0.2) (layer "B.Cu") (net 3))
 (segment (start 103.925 57.2) (end 111.095 64.37) (width 0.2) (layer "F.Cu") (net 1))
 (segment (start 120.13 64.87) (end 121.623985 66.363985) (width 0.2) (layer "F.Cu") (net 1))
 (segment (start 143.277749 68.903985) (end 144.904095 68.903985) (width 0.2) (layer "F.Cu") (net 1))
 (segment (start 123.863985 66.363985) (end 124.584095 67.084095) (width 0.2) (layer "F.Cu") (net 1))
 (segment (start 124.584095 67.084095) (end 124.584095 68.903985) (width 0.2) (layer "F.Cu") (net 1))
 (segment (start 142.124095 66.544095) (end 142.124095 67.750331) (width 0.2) (layer "F.Cu") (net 1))
 (segment (start 121.623985 66.363985) (end 123.863985 66.363985) (width 0.2) (layer "F.Cu") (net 1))
 (segment (start 144.904095 68.903985) (end 146.054095 70.053985) (width 0.2) (layer "F.Cu") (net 1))
 (segment (start 119.63 64.37) (end 120.13 64.87) (width 0.2) (layer "F.Cu") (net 1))
 (segment (start 138.32 62.74) (end 142.124095 66.544095) (width 0.2) (layer "F.Cu") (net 1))
 (segment (start 118 62.74) (end 119.63 64.37) (width 0.2) (layer "F.Cu") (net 1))
 (segment (start 208 63.7) (end 201.646015 70.053985) (width 0.2) (layer "F.Cu") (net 1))
 (segment (start 124.584095 68.903985) (end 125.734095 70.053985) (width 0.2) (layer "F.Cu") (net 1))
 (segment (start 142.124095 67.750331) (end 143.277749 68.903985) (width 0.2) (layer "F.Cu") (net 1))
 (segment (start 111.095 64.37) (end 119.63 64.37) (width 0.2) (layer "F.Cu") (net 1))
 (segment (start 117 66) (end 117 66.39989) (width 0.2) (layer "F.Cu") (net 17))
 (segment (start 101.385 57.2) (end 101.385 58.830685) (width 0.2) (layer "F.Cu") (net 17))
 (segment (start 108.054315 65.5) (end 116.5 65.5) (width 0.2) (layer "F.Cu") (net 17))
 (segment (start 101.385 58.830685) (end 108.054315 65.5) (width 0.2) (layer "F.Cu") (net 17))
 (segment (start 117 66.39989) (end 118.114095 67.513985) (width 0.2) (layer "F.Cu") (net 17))
 (segment (start 116.5 65.5) (end 117 66) (width 0.2) (layer "F.Cu") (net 17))
 (segment (start 91.225 57.2) (end 100.334095 66.309095) (width 0.2) (layer "F.Cu") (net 13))
 (segment (start 100.334095 66.309095) (end 100.334095 67.513985) (width 0.2) (layer "F.Cu") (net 13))
 (segment (start 118 57.5) (end 151.5 57.5) (width 0.2) (layer "F.Cu") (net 2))
 (segment (start 144 67.02808) (end 143.514095 67.513985) (width 0.2) (layer "F.Cu") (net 2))
 (segment (start 150.5 65) (end 150 65.5) (width 0.2) (layer "F.Cu") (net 2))
 (segment (start 118 60.2) (end 118 57.5) (width 0.2) (layer "F.Cu") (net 2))
 (segment (start 110.2 57.2) (end 112 59) (width 0.2) (layer "F.Cu") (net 2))
 (segment (start 149.5 67) (end 148.986015 67.513985) (width 0.2) (layer "F.Cu") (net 2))
 (segment (start 150 67) (end 149.5 67) (width 0.2) (layer "F.Cu") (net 2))
 (segment (start 144 65.5) (end 144 67.02808) (width 0.2) (layer "F.Cu") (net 2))
 (segment (start 151.5 57.5) (end 151.5 65.5) (width 0.2) (layer "F.Cu") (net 2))
 (segment (start 106.465 57.2) (end 110.2 57.2) (width 0.2) (layer "F.Cu") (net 2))
 (segment (start 120.5 58.5) (end 150.5 58.5) (width 0.2) (layer "F.Cu") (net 2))
 (segment (start 120.54 58.54) (end 120.5 58.5) (width 0.2) (layer "F.Cu") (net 2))
 (segment (start 150.5 58.5) (end 150.5 65) (width 0.2) (layer "F.Cu") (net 2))
 (segment (start 116.8 59) (end 118 60.2) (width 0.2) (layer "F.Cu") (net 2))
 (segment (start 151.5 65.5) (end 150 67) (width 0.2) (layer "F.Cu") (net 2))
 (segment (start 148.986015 67.513985) (end 146.054095 67.513985) (width 0.2) (layer "F.Cu") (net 2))
 (segment (start 120.54 60.2) (end 120.54 58.54) (width 0.2) (layer "F.Cu") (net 2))
 (segment (start 112 59) (end 116.8 59) (width 0.2) (layer "F.Cu") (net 2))
 (segment (start 150 65.5) (end 144 65.5) (width 0.2) (layer "F.Cu") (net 2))
 (segment (start 107.954095 67.374095) (end 107.954095 67.513985) (width 0.2) (layer "F.Cu") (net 15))
 (segment (start 97.455 58.35) (end 98.79011 58.35) (width 0.2) (layer "F.Cu") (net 15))
 (segment (start 96.305 57.2) (end 97.455 58.35) (width 0.2) (layer "F.Cu") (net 15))
 (segment (start 98.79011 58.35) (end 107.954095 67.513985) (width 0.2) (layer "F.Cu") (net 15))
 (segment (start 108.008985 66.363985) (end 114.424095 66.363985) (width 0.2) (layer "F.Cu") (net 16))
 (segment (start 114.424095 66.363985) (end 115.574095 67.513985) (width 0.2) (layer "F.Cu") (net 16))
 (segment (start 98.845 57.2) (end 108.008985 66.363985) (width 0.2) (layer "F.Cu") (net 16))
 (segment (start 101.324095 71.603985) (end 102.874095 70.053985) (width 0.2) (layer "F.Cu") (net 10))
 (segment (start 95.176219 71.603985) (end 101.324095 71.603985) (width 0.2) (layer "F.Cu") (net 10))
 (segment (start 83.605 60.032766) (end 95.176219 71.603985) (width 0.2) (layer "F.Cu") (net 10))
 (segment (start 83.605 57.2) (end 83.605 60.032766) (width 0.2) (layer "F.Cu") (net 10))
 (segment (start 88.685 58.40489) (end 97.794095 67.513985) (width 0.2) (layer "F.Cu") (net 12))
 (segment (start 88.685 57.2) (end 88.685 58.40489) (width 0.2) (layer "F.Cu") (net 12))
 (segment (start 102.874095 66.309095) (end 102.874095 67.513985) (width 0.2) (layer "F.Cu") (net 14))
 (segment (start 93.765 57.2) (end 102.874095 66.309095) (width 0.2) (layer "F.Cu") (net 14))
 (segment (start 208 66.24) (end 202.636015 71.603985) (width 0.2) (layer "F.Cu") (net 18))
 (segment (start 122.204095 71.603985) (end 120.654095 70.053985) (width 0.2) (layer "F.Cu") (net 18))
 (segment (start 180.083462 60.64) (end 167.523462 73.2) (width 0.2) (layer "B.Cu") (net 4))
 (segment (start 143.514095 73.085905) (end 143.514095 70.053985) (width 0.2) (layer "B.Cu") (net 4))
 (segment (start 167.523462 73.2) (end 143.4 73.2) (width 0.2) (layer "B.Cu") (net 4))
 (segment (start 143.4 73.2) (end 143.514095 73.085905) (width 0.2) (layer "B.Cu") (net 4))
 (segment (start 180.083462 63.18) (end 169.662462 73.601) (width 0.2) (layer "B.Cu") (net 5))
 (segment (start 143.2339 73.601) (end 140.974095 71.341195) (width 0.2) (layer "B.Cu") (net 5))
 (segment (start 169.662462 73.601) (end 143.2339 73.601) (width 0.2) (layer "B.Cu") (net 5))
 (segment (start 140.974095 71.341195) (end 140.974095 70.053985) (width 0.2) (layer "B.Cu") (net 5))
 (segment (start 81.065 58.402081) (end 94.666904 72.003985) (width 0.2) (layer "F.Cu") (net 9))
 (segment (start 122 69.773544) (end 122 70.486236) (width 0.2) (layer "F.Cu") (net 9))
 (segment (start 81.065 57.2) (end 81.065 58.402081) (width 0.2) (layer "F.Cu") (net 9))
 (segment (start 86.145 60.031236) (end 97.317749 71.203985) (width 0.2) (layer "F.Cu") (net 9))
 (segment (start 94.666904 72.003985) (end 102.996015 72.003985) (width 0.2) (layer "F.Cu") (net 9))
 (segment (start 121.130441 68.903985) (end 122 69.773544) (width 0.2) (layer "F.Cu") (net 9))
 (segment (start 112.673764 73.86) (end 109.344095 70.530331) (width 0.2) (layer "F.Cu") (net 9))
 (segment (start 102.996015 72.003985) (end 104.264095 70.735905) (width 0.2) (layer "F.Cu") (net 9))
 (segment (start 99.184095 71.203985) (end 97.317749 71.203985) (width 0.2) (layer "F.Cu") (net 9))
 (segment (start 100.334095 70.053985) (end 99.184095 71.203985) (width 0.2) (layer "F.Cu") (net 9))
 (segment (start 104.937749 68.903985) (end 109.5 68.903985) (width 0.2) (layer "F.Cu") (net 9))
 (segment (start 131.796015 71.203985) (end 132.204095 70.795905) (width 0.2) (layer "F.Cu") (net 9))
 (segment (start 104.264095 70.735905) (end 104.264095 69.577639) (width 0.2) (layer "F.Cu") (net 9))
 (segment (start 109.344095 70.530331) (end 109.344095 69.05989) (width 0.2) (layer "F.Cu") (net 9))
 (segment (start 109.5 68.903985) (end 121.130441 68.903985) (width 0.2) (layer "F.Cu") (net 9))
 (segment (start 122 70.486236) (end 122.717749 71.203985) (width 0.2) (layer "F.Cu") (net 9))
 (segment (start 104.264095 69.577639) (end 104.937749 68.903985) (width 0.2) (layer "F.Cu") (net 9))
 (segment (start 86.145 57.2) (end 86.145 60.031236) (width 0.2) (layer "F.Cu") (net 9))
 (segment (start 132.204095 70.795905) (end 132.204095 68.663985) (width 0.2) (layer "F.Cu") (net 9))
 (segment (start 109.344095 69.05989) (end 109.5 68.903985) (width 0.2) (layer "F.Cu") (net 9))
 (segment (start 122.717749 71.203985) (end 131.796015 71.203985) (width 0.2) (layer "F.Cu") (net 9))
 (segment (start 132.204095 68.663985) (end 133.354095 67.513985) (width 0.2) (layer "F.Cu") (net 9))
 (segment (start 105.414095 70.053985) (end 111.76011 76.4) (width 0.2) (layer "F.Cu") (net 22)))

